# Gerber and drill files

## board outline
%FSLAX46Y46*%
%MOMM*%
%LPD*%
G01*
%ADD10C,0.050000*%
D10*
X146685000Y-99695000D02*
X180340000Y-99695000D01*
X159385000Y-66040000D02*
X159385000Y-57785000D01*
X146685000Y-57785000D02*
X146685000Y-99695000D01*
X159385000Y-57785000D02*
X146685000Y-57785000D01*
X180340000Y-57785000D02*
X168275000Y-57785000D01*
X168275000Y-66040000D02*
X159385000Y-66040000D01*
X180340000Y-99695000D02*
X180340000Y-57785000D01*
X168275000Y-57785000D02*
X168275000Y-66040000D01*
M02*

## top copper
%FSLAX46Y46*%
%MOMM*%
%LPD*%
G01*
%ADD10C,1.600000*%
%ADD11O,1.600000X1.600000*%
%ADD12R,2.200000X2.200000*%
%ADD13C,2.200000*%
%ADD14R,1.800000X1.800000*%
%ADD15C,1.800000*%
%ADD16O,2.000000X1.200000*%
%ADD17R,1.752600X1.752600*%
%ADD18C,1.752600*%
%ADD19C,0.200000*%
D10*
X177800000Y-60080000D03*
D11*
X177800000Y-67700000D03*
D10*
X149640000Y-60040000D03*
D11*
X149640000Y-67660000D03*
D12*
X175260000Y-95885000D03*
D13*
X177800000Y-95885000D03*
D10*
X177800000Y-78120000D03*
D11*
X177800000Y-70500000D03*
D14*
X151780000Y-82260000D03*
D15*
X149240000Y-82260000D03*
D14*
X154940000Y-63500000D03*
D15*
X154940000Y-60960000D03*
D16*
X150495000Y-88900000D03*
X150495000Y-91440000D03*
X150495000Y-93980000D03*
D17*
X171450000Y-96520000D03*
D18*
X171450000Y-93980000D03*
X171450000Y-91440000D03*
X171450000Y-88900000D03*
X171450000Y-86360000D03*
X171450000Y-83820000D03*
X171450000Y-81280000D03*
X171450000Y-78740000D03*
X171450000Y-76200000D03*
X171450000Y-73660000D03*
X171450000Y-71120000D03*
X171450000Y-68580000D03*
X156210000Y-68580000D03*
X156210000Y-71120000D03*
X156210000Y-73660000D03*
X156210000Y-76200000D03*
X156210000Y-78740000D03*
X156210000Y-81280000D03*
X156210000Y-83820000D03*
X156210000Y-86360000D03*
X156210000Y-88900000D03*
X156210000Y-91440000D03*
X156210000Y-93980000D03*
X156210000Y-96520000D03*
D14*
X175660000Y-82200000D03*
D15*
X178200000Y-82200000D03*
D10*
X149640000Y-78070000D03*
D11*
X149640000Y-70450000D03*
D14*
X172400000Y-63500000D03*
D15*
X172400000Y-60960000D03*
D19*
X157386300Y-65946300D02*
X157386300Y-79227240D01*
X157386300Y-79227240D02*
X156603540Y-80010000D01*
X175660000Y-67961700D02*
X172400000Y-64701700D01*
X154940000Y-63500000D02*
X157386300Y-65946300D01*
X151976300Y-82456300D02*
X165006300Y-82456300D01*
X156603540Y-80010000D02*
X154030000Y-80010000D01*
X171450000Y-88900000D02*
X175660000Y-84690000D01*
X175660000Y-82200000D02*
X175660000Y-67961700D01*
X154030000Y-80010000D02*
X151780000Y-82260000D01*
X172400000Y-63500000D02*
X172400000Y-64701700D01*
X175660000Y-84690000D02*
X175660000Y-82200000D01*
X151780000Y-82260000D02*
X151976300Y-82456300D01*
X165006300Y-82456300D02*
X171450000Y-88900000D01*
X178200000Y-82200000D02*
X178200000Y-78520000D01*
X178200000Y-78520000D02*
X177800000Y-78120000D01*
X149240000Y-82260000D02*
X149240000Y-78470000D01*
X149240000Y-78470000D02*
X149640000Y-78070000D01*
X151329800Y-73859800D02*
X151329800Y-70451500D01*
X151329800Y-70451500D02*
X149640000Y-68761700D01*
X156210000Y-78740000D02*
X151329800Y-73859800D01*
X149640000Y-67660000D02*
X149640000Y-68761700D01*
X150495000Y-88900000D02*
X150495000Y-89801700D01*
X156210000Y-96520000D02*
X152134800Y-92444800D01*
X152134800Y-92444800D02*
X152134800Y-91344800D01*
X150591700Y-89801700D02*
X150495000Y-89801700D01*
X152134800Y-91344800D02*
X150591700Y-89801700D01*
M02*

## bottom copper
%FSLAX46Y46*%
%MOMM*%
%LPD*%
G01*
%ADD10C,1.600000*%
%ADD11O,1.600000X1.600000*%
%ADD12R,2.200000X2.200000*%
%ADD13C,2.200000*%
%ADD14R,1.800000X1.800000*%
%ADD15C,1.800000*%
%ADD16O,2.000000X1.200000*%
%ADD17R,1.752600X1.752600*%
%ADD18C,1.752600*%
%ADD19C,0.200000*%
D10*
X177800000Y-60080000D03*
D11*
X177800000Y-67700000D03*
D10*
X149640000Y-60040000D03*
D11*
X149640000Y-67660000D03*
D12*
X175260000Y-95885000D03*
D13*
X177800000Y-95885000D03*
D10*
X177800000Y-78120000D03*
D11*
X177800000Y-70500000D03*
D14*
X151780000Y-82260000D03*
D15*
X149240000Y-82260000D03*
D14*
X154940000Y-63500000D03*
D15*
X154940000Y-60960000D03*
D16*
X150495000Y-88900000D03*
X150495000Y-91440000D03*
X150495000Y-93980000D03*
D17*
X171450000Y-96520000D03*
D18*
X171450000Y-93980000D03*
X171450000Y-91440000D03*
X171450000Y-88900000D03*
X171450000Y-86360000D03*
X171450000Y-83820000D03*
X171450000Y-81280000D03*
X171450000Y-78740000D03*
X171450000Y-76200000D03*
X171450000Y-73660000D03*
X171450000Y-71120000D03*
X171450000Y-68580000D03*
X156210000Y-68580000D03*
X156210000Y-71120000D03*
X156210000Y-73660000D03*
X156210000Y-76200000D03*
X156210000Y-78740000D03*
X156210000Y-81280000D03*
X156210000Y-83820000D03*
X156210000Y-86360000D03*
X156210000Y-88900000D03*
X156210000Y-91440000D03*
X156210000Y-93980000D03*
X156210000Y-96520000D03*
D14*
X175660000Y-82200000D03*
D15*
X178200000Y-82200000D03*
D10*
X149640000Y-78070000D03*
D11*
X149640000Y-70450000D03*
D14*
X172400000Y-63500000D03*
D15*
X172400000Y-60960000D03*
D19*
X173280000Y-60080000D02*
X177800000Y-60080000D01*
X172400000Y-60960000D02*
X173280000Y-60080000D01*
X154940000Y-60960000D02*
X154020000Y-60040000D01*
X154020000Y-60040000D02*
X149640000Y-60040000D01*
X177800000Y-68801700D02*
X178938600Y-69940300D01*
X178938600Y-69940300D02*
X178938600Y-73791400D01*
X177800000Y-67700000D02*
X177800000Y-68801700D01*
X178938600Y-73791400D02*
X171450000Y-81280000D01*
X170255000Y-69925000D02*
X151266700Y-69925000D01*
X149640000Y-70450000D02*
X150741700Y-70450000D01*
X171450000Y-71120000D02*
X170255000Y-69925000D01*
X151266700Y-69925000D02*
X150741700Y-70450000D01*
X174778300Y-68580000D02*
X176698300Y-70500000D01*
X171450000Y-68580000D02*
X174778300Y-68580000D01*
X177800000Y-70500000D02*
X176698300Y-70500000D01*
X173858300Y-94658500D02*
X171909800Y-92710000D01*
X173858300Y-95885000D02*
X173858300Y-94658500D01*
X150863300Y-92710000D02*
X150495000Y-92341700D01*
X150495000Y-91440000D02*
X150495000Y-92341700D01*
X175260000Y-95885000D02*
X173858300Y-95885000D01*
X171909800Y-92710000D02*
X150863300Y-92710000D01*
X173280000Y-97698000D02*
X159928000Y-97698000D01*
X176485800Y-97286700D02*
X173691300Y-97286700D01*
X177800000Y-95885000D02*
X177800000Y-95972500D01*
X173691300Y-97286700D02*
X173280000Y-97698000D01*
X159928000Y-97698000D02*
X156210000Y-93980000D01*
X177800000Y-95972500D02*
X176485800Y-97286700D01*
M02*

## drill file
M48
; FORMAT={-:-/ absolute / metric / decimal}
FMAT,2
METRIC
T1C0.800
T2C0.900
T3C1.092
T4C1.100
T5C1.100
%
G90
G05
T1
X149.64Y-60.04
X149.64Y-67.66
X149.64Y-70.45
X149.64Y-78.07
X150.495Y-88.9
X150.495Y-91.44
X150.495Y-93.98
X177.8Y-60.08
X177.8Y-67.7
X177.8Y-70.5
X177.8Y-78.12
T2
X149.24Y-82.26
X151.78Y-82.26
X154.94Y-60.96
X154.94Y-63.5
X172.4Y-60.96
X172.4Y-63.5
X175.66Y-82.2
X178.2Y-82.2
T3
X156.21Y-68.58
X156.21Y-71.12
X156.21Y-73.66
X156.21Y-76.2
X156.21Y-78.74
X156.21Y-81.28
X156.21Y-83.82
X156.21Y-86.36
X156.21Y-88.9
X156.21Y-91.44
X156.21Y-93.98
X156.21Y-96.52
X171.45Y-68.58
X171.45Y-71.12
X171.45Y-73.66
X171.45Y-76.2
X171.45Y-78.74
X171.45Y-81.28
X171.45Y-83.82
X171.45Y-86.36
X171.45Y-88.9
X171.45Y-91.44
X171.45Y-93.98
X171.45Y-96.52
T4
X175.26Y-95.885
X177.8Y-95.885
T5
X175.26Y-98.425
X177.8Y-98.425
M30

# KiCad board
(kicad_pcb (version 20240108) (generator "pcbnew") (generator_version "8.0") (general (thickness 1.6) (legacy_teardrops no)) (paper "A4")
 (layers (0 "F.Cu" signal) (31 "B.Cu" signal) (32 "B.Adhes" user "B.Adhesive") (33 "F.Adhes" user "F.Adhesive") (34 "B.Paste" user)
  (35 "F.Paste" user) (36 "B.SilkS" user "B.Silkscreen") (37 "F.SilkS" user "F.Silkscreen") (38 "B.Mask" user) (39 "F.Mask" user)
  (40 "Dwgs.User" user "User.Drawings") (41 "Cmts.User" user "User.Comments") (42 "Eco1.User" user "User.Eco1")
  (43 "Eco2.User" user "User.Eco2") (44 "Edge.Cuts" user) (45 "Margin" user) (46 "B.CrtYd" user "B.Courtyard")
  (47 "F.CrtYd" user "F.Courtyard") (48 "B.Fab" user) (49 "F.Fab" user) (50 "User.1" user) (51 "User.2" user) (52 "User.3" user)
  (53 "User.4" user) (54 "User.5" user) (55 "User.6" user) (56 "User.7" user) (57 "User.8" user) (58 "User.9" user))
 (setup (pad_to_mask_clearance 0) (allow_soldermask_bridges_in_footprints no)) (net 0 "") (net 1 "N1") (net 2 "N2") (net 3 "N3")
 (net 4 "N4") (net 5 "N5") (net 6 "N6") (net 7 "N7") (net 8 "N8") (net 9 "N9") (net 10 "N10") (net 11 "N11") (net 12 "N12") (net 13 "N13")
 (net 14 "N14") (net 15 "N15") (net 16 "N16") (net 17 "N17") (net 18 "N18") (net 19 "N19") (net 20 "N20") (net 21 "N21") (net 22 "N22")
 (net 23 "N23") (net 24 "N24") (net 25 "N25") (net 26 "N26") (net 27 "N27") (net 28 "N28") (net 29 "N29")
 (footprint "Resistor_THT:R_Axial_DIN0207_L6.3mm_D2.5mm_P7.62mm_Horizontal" (layer "F.Cu") (at 177.8 60.08 -90)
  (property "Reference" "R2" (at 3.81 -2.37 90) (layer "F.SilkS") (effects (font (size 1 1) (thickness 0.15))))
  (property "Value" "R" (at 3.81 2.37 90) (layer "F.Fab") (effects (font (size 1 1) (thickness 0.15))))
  (pad "1" thru_hole circle (at 0 0 270) (size 1.6 1.6) (drill 0.8) (layers "*.Cu" "*.Mask") (remove_unused_layers no) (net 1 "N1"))
  (pad "2" thru_hole oval (at 7.62 0 270) (size 1.6 1.6) (drill 0.8) (layers "*.Cu" "*.Mask") (remove_unused_layers no) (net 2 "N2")))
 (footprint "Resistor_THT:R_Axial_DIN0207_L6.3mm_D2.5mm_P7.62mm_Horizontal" (layer "F.Cu") (at 149.64 60.04 -90)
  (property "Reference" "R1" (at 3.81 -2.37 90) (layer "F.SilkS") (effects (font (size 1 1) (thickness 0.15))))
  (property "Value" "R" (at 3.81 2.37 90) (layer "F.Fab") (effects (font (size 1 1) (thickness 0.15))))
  (pad "1" thru_hole circle (at 0 0 270) (size 1.6 1.6) (drill 0.8) (layers "*.Cu" "*.Mask") (remove_unused_layers no) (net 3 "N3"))
  (pad "2" thru_hole oval (at 7.62 0 270) (size 1.6 1.6) (drill 0.8) (layers "*.Cu" "*.Mask") (remove_unused_layers no) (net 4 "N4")))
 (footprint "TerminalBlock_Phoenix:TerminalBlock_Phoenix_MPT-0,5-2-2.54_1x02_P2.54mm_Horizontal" (layer "F.Cu") (at 175.26 95.885)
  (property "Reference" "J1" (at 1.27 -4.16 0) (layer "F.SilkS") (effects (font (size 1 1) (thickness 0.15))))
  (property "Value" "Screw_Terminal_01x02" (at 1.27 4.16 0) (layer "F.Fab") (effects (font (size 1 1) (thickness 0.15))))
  (pad "" np_thru_hole circle (at 0 2.54) (size 1.1 1.1) (drill 1.1) (layers "*.Cu" "*.Mask"))
  (pad "" np_thru_hole circle (at 2.54 2.54) (size 1.1 1.1) (drill 1.1) (layers "*.Cu" "*.Mask"))
  (pad "1" thru_hole rect (at 0 0) (size 2.2 2.2) (drill 1.1) (layers "*.Cu" "*.Mask") (remove_unused_layers no) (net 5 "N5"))
  (pad "2" thru_hole circle (at 2.54 0) (size 2.2 2.2) (drill 1.1) (layers "*.Cu" "*.Mask") (remove_unused_layers no) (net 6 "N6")))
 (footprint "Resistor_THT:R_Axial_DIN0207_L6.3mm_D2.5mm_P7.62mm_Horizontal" (layer "F.Cu") (at 177.8 78.12 90)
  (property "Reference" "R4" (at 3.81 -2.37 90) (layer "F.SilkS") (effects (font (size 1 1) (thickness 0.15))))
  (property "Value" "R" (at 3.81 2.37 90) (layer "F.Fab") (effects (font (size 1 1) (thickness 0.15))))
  (pad "1" thru_hole circle (at 0 0 90) (size 1.6 1.6) (drill 0.8) (layers "*.Cu" "*.Mask") (remove_unused_layers no) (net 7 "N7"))
  (pad "2" thru_hole oval (at 7.62 0 90) (size 1.6 1.6) (drill 0.8) (layers "*.Cu" "*.Mask") (remove_unused_layers no) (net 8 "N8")))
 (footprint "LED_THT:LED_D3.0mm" (layer "F.Cu") (at 151.78 82.26 180)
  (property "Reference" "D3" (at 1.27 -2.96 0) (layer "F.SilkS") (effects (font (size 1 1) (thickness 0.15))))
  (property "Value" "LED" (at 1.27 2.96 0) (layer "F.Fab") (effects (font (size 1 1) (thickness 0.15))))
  (pad "1" thru_hole rect (at 0 0 180) (size 1.8 1.8) (drill 0.9) (layers "*.Cu" "*.Mask") (remove_unused_layers no) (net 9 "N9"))
  (pad "2" thru_hole circle (at 2.54 0 180) (size 1.8 1.8) (drill 0.9) (layers "*.Cu" "*.Mask") (remove_unused_layers no) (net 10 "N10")))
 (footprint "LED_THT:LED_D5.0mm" (layer "F.Cu") (at 154.94 63.5 90)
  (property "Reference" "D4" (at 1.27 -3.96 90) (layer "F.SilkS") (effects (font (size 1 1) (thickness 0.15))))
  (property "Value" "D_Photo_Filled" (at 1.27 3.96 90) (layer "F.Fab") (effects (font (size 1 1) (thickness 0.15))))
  (pad "1" thru_hole rect (at 0 0 90) (size 1.8 1.8) (drill 0.9) (layers "*.Cu" "*.Mask") (remove_unused_layers no) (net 9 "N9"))
  (pad "2" thru_hole circle (at 2.54 0 90) (size 1.8 1.8) (drill 0.9) (layers "*.Cu" "*.Mask") (remove_unused_layers no) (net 3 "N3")))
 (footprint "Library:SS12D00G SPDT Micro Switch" (layer "F.Cu") (at 150.495 91.44 -90)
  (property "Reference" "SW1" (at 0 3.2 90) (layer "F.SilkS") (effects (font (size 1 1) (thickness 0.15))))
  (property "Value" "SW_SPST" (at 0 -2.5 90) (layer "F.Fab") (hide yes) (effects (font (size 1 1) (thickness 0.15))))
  (pad "1" thru_hole oval (at -2.54 0 270) (size 1.2 2) (drill 0.8) (layers "*.Cu" "*.Mask") (remove_unused_layers no) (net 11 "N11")
   (thermal_bridge_angle 45))
  (pad "2" thru_hole oval (at 0 0 270) (size 1.2 2) (drill 0.8) (layers "*.Cu" "*.Mask") (remove_unused_layers no) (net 5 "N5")
   (thermal_bridge_angle 45))
  (pad "3" thru_hole oval (at 2.54 0 270) (size 1.2 2) (drill 0.8) (layers "*.Cu" "*.Mask") (remove_unused_layers no)
   (thermal_bridge_angle 45)))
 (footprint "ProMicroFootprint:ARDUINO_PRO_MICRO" (layer "F.Cu") (at 163.83 82.55 90)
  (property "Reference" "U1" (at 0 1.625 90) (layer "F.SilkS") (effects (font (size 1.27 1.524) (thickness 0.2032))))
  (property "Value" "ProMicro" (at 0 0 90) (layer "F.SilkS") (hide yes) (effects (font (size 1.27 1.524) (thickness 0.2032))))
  (pad "1" thru_hole rect (at -13.97 7.62 90) (size 1.7526 1.7526) (drill 1.0922) (layers "*.Cu" "*.SilkS" "*.Mask")
   (remove_unused_layers no) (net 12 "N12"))
  (pad "2" thru_hole circle (at -11.43 7.62 90) (size 1.7526 1.7526) (drill 1.0922) (layers "*.Cu" "*.SilkS" "*.Mask")
   (remove_unused_layers no) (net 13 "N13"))
  (pad "3" thru_hole circle (at -8.89 7.62 90) (size 1.7526 1.7526) (drill 1.0922) (layers "*.Cu" "*.SilkS" "*.Mask")
   (remove_unused_layers no) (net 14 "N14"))
  (pad "4" thru_hole circle (at -6.35 7.62 90) (size 1.7526 1.7526) (drill 1.0922) (layers "*.Cu" "*.SilkS" "*.Mask")
   (remove_unused_layers no) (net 9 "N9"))
  (pad "5" thru_hole circle (at -3.81 7.62 90) (size 1.7526 1.7526) (drill 1.0922) (layers "*.Cu" "*.SilkS" "*.Mask")
   (remove_unused_layers no) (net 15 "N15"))
  (pad "6" thru_hole circle (at -1.27 7.62 90) (size 1.7526 1.7526) (drill 1.0922) (layers "*.Cu" "*.SilkS" "*.Mask")
   (remove_unused_layers no) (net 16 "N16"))
  (pad "7" thru_hole circle (at 1.27 7.62 90) (size 1.7526 1.7526) (drill 1.0922) (layers "*.Cu" "*.SilkS" "*.Mask")
   (remove_unused_layers no) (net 2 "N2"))
  (pad "8" thru_hole circle (at 3.81 7.62 90) (size 1.7526 1.7526) (drill 1.0922) (layers "*.Cu" "*.SilkS" "*.Mask")
   (remove_unused_layers no) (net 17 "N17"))
  (pad "9" thru_hole circle (at 6.35 7.62 90) (size 1.7526 1.7526) (drill 1.0922) (layers "*.Cu" "*.SilkS" "*.Mask")
   (remove_unused_layers no) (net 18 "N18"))
  (pad "10" thru_hole circle (at 8.89 7.62 90) (size 1.7526 1.7526) (drill 1.0922) (layers "*.Cu" "*.SilkS" "*.Mask")
   (remove_unused_layers no) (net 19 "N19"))
  (pad "11" thru_hole circle (at 11.43 7.62 90) (size 1.7526 1.7526) (drill 1.0922) (layers "*.Cu" "*.SilkS" "*.Mask")
   (remove_unused_layers no) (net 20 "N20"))
  (pad "12" thru_hole circle (at 13.97 7.62 90) (size 1.7526 1.7526) (drill 1.0922) (layers "*.Cu" "*.SilkS" "*.Mask")
   (remove_unused_layers no) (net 8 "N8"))
  (pad "13" thru_hole circle (at 13.97 -7.62 90) (size 1.7526 1.7526) (drill 1.0922) (layers "*.Cu" "*.SilkS" "*.Mask")
   (remove_unused_layers no) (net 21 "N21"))
  (pad "14" thru_hole circle (at 11.43 -7.62 90) (size 1.7526 1.7526) (drill 1.0922) (layers "*.Cu" "*.SilkS" "*.Mask")
   (remove_unused_layers no) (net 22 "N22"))
  (pad "15" thru_hole circle (at 8.89 -7.62 90) (size 1.7526 1.7526) (drill 1.0922) (layers "*.Cu" "*.SilkS" "*.Mask")
   (remove_unused_layers no) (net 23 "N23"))
  (pad "16" thru_hole circle (at 6.35 -7.62 90) (size 1.7526 1.7526) (drill 1.0922) (layers "*.Cu" "*.SilkS" "*.Mask")
   (remove_unused_layers no) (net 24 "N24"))
  (pad "17" thru_hole circle (at 3.81 -7.62 90) (size 1.7526 1.7526) (drill 1.0922) (layers "*.Cu" "*.SilkS" "*.Mask")
   (remove_unused_layers no) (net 4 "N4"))
  (pad "18" thru_hole circle (at 1.27 -7.62 90) (size 1.7526 1.7526) (drill 1.0922) (layers "*.Cu" "*.SilkS" "*.Mask")
   (remove_unused_layers no) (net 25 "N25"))
  (pad "19" thru_hole circle (at -1.27 -7.62 90) (size 1.7526 1.7526) (drill 1.0922) (layers "*.Cu" "*.SilkS" "*.Mask")
   (remove_unused_layers no) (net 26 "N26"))
  (pad "20" thru_hole circle (at -3.81 -7.62 90) (size 1.7526 1.7526) (drill 1.0922) (layers "*.Cu" "*.SilkS" "*.Mask")
   (remove_unused_layers no) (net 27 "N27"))
  (pad "21" thru_hole circle (at -6.35 -7.62 90) (size 1.7526 1.7526) (drill 1.0922) (layers "*.Cu" "*.SilkS" "*.Mask")
   (remove_unused_layers no) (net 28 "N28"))
  (pad "22" thru_hole circle (at -8.89 -7.62 90) (size 1.7526 1.7526) (drill 1.0922) (layers "*.Cu" "*.SilkS" "*.Mask")
   (remove_unused_layers no) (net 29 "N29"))
  (pad "23" thru_hole circle (at -11.43 -7.62 90) (size 1.7526 1.7526) (drill 1.0922) (layers "*.Cu" "*.SilkS" "*.Mask")
   (remove_unused_layers no) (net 6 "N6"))
  (pad "24" thru_hole circle (at -13.97 -7.62 90) (size 1.7526 1.7526) (drill 1.0922) (layers "*.Cu" "*.SilkS" "*.Mask")
   (remove_unused_layers no) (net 11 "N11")))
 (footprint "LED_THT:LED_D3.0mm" (layer "F.Cu") (at 175.66 82.2)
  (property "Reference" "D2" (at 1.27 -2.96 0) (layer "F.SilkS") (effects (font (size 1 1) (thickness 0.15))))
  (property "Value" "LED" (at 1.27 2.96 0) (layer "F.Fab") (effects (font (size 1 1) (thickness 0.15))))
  (pad "1" thru_hole rect (at 0 0) (size 1.8 1.8) (drill 0.9) (layers "*.Cu" "*.Mask") (remove_unused_layers no) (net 9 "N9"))
  (pad "2" thru_hole circle (at 2.54 0) (size 1.8 1.8) (drill 0.9) (layers "*.Cu" "*.Mask") (remove_unused_layers no) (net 7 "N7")))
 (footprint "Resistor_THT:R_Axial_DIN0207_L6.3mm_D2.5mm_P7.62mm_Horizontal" (layer "F.Cu") (at 149.64 78.07 90)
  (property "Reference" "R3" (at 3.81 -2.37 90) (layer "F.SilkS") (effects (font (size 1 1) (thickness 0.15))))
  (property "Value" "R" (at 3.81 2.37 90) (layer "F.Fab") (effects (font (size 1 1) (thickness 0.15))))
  (pad "1" thru_hole circle (at 0 0 90) (size 1.6 1.6) (drill 0.8) (layers "*.Cu" "*.Mask") (remove_unused_layers no) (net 10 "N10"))
  (pad "2" thru_hole oval (at 7.62 0 90) (size 1.6 1.6) (drill 0.8) (layers "*.Cu" "*.Mask") (remove_unused_layers no) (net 20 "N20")))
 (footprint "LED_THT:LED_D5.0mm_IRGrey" (layer "F.Cu") (at 172.4 63.5 90)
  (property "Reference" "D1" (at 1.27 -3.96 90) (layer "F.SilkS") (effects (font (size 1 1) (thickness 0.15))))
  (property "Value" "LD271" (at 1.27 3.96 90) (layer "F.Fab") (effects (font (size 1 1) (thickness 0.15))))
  (pad "1" thru_hole rect (at 0 0 90) (size 1.8 1.8) (drill 0.9) (layers "*.Cu" "*.Mask") (remove_unused_layers no) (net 9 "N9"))
  (pad "2" thru_hole circle (at 2.54 0 90) (size 1.8 1.8) (drill 0.9) (layers "*.Cu" "*.Mask") (remove_unused_layers no) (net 1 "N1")))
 (gr_line (start 146.685 99.695) (end 180.34 99.695) (stroke (width 0.05) (type default)) (layer "Edge.Cuts"))
 (gr_line (start 159.385 66.04) (end 159.385 57.785) (stroke (width 0.05) (type default)) (layer "Edge.Cuts"))
 (gr_line (start 146.685 57.785) (end 146.685 99.695) (stroke (width 0.05) (type default)) (layer "Edge.Cuts"))
 (gr_line (start 159.385 57.785) (end 146.685 57.785) (stroke (width 0.05) (type default)) (layer "Edge.Cuts"))
 (gr_line (start 180.34 57.785) (end 168.275 57.785) (stroke (width 0.05) (type default)) (layer "Edge.Cuts"))
 (gr_line (start 168.275 66.04) (end 159.385 66.04) (stroke (width 0.05) (type default)) (layer "Edge.Cuts"))
 (gr_line (start 180.34 99.695) (end 180.34 57.785) (stroke (width 0.05) (type default)) (layer "Edge.Cuts"))
 (gr_line (start 168.275 57.785) (end 168.275 66.04) (stroke (width 0.05) (type default)) (layer "Edge.Cuts"))
 (segment (start 157.3863 65.9463) (end 157.3863 79.22724) (width 0.2) (layer "F.Cu") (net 9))
 (segment (start 157.3863 79.22724) (end 156.60354 80.01) (width 0.2) (layer "F.Cu") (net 9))
 (segment (start 175.66 67.9617) (end 172.4 64.7017) (width 0.2) (layer "F.Cu") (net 9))
 (segment (start 154.94 63.5) (end 157.3863 65.9463) (width 0.2) (layer "F.Cu") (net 9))
 (segment (start 151.9763 82.4563) (end 165.0063 82.4563) (width 0.2) (layer "F.Cu") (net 9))
 (segment (start 156.60354 80.01) (end 154.03 80.01) (width 0.2) (layer "F.Cu") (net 9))
 (segment (start 171.45 88.9) (end 175.66 84.69) (width 0.2) (layer "F.Cu") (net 9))
 (segment (start 175.66 82.2) (end 175.66 67.9617) (width 0.2) (layer "F.Cu") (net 9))
 (segment (start 154.03 80.01) (end 151.78 82.26) (width 0.2) (layer "F.Cu") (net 9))
 (segment (start 172.4 63.5) (end 172.4 64.7017) (width 0.2) (layer "F.Cu") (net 9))
 (segment (start 175.66 84.69) (end 175.66 82.2) (width 0.2) (layer "F.Cu") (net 9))
 (segment (start 151.78 82.26) (end 151.9763 82.4563) (width 0.2) (layer "F.Cu") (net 9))
 (segment (start 165.0063 82.4563) (end 171.45 88.9) (width 0.2) (layer "F.Cu") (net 9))
 (segment (start 173.28 60.08) (end 177.8 60.08) (width 0.2) (layer "B.Cu") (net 1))
 (segment (start 172.4 60.96) (end 173.28 60.08) (width 0.2) (layer "B.Cu") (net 1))
 (segment (start 178.2 82.2) (end 178.2 78.52) (width 0.2) (layer "F.Cu") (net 7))
 (segment (start 178.2 78.52) (end 177.8 78.12) (width 0.2) (layer "F.Cu") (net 7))
 (segment (start 149.24 82.26) (end 149.24 78.47) (width 0.2) (layer "F.Cu") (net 10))
 (segment (start 149.24 78.47) (end 149.64 78.07) (width 0.2) (layer "F.Cu") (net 10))
 (segment (start 154.94 60.96) (end 154.02 60.04) (width 0.2) (layer "B.Cu") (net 3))
 (segment (start 154.02 60.04) (end 149.64 60.04) (width 0.2) (layer "B.Cu") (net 3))
 (segment (start 151.3298 73.8598) (end 151.3298 70.4515) (width 0.2) (layer "F.Cu") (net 4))
 (segment (start 151.3298 70.4515) (end 149.64 68.7617) (width 0.2) (layer "F.Cu") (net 4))
 (segment (start 156.21 78.74) (end 151.3298 73.8598) (width 0.2) (layer "F.Cu") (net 4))
 (segment (start 149.64 67.66) (end 149.64 68.7617) (width 0.2) (layer "F.Cu") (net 4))
 (segment (start 177.8 68.8017) (end 178.9386 69.9403) (width 0.2) (layer "B.Cu") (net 2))
 (segment (start 178.9386 69.9403) (end 178.9386 73.7914) (width 0.2) (layer "B.Cu") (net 2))
 (segment (start 177.8 67.7) (end 177.8 68.8017) (width 0.2) (layer "B.Cu") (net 2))
 (segment (start 178.9386 73.7914) (end 171.45 81.28) (width 0.2) (layer "B.Cu") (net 2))
 (segment (start 170.255 69.925) (end 151.2667 69.925) (width 0.2) (layer "B.Cu") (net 20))
 (segment (start 149.64 70.45) (end 150.7417 70.45) (width 0.2) (layer "B.Cu") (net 20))
 (segment (start 171.45 71.12) (end 170.255 69.925) (width 0.2) (layer "B.Cu") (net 20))
 (segment (start 151.2667 69.925) (end 150.7417 70.45) (width 0.2) (layer "B.Cu") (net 20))
 (segment (start 174.7783 68.58) (end 176.6983 70.5) (width 0.2) (layer "B.Cu") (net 8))
 (segment (start 171.45 68.58) (end 174.7783 68.58) (width 0.2) (layer "B.Cu") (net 8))
 (segment (start 177.8 70.5) (end 176.6983 70.5) (width 0.2) (layer "B.Cu") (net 8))
 (segment (start 150.495 88.9) (end 150.495 89.8017) (width 0.2) (layer "F.Cu") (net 11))
 (segment (start 156.21 96.52) (end 152.1348 92.4448) (width 0.2) (layer "F.Cu") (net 11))
 (segment (start 152.1348 92.4448) (end 152.1348 91.3448) (width 0.2) (layer "F.Cu") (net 11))
 (segment (start 150.5917 89.8017) (end 150.495 89.8017) (width 0.2) (layer "F.Cu") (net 11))
 (segment (start 152.1348 91.3448) (end 150.5917 89.8017) (width 0.2) (layer "F.Cu") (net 11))
 (segment (start 173.8583 94.6585) (end 171.9098 92.71) (width 0.2) (layer "B.Cu") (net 5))
 (segment (start 173.8583 95.885) (end 173.8583 94.6585) (width 0.2) (layer "B.Cu") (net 5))
 (segment (start 150.8633 92.71) (end 150.495 92.3417) (width 0.2) (layer "B.Cu") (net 5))
 (segment (start 150.495 91.44) (end 150.495 92.3417) (width 0.2) (layer "B.Cu") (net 5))
 (segment (start 175.26 95.885) (end 173.8583 95.885) (width 0.2) (layer "B.Cu") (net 5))
 (segment (start 171.9098 92.71) (end 150.8633 92.71) (width 0.2) (layer "B.Cu") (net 5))
 (segment (start 173.28 97.698) (end 159.928 97.698) (width 0.2) (layer "B.Cu") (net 6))
 (segment (start 176.4858 97.2867) (end 173.6913 97.2867) (width 0.2) (layer "B.Cu") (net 6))
 (segment (start 177.8 95.885) (end 177.8 95.9725) (width 0.2) (layer "B.Cu") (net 6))
 (segment (start 173.6913 97.2867) (end 173.28 97.698) (width 0.2) (layer "B.Cu") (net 6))
 (segment (start 159.928 97.698) (end 156.21 93.98) (width 0.2) (layer "B.Cu") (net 6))
 (segment (start 177.8 95.9725) (end 176.4858 97.2867) (width 0.2) (layer "B.Cu") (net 6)))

